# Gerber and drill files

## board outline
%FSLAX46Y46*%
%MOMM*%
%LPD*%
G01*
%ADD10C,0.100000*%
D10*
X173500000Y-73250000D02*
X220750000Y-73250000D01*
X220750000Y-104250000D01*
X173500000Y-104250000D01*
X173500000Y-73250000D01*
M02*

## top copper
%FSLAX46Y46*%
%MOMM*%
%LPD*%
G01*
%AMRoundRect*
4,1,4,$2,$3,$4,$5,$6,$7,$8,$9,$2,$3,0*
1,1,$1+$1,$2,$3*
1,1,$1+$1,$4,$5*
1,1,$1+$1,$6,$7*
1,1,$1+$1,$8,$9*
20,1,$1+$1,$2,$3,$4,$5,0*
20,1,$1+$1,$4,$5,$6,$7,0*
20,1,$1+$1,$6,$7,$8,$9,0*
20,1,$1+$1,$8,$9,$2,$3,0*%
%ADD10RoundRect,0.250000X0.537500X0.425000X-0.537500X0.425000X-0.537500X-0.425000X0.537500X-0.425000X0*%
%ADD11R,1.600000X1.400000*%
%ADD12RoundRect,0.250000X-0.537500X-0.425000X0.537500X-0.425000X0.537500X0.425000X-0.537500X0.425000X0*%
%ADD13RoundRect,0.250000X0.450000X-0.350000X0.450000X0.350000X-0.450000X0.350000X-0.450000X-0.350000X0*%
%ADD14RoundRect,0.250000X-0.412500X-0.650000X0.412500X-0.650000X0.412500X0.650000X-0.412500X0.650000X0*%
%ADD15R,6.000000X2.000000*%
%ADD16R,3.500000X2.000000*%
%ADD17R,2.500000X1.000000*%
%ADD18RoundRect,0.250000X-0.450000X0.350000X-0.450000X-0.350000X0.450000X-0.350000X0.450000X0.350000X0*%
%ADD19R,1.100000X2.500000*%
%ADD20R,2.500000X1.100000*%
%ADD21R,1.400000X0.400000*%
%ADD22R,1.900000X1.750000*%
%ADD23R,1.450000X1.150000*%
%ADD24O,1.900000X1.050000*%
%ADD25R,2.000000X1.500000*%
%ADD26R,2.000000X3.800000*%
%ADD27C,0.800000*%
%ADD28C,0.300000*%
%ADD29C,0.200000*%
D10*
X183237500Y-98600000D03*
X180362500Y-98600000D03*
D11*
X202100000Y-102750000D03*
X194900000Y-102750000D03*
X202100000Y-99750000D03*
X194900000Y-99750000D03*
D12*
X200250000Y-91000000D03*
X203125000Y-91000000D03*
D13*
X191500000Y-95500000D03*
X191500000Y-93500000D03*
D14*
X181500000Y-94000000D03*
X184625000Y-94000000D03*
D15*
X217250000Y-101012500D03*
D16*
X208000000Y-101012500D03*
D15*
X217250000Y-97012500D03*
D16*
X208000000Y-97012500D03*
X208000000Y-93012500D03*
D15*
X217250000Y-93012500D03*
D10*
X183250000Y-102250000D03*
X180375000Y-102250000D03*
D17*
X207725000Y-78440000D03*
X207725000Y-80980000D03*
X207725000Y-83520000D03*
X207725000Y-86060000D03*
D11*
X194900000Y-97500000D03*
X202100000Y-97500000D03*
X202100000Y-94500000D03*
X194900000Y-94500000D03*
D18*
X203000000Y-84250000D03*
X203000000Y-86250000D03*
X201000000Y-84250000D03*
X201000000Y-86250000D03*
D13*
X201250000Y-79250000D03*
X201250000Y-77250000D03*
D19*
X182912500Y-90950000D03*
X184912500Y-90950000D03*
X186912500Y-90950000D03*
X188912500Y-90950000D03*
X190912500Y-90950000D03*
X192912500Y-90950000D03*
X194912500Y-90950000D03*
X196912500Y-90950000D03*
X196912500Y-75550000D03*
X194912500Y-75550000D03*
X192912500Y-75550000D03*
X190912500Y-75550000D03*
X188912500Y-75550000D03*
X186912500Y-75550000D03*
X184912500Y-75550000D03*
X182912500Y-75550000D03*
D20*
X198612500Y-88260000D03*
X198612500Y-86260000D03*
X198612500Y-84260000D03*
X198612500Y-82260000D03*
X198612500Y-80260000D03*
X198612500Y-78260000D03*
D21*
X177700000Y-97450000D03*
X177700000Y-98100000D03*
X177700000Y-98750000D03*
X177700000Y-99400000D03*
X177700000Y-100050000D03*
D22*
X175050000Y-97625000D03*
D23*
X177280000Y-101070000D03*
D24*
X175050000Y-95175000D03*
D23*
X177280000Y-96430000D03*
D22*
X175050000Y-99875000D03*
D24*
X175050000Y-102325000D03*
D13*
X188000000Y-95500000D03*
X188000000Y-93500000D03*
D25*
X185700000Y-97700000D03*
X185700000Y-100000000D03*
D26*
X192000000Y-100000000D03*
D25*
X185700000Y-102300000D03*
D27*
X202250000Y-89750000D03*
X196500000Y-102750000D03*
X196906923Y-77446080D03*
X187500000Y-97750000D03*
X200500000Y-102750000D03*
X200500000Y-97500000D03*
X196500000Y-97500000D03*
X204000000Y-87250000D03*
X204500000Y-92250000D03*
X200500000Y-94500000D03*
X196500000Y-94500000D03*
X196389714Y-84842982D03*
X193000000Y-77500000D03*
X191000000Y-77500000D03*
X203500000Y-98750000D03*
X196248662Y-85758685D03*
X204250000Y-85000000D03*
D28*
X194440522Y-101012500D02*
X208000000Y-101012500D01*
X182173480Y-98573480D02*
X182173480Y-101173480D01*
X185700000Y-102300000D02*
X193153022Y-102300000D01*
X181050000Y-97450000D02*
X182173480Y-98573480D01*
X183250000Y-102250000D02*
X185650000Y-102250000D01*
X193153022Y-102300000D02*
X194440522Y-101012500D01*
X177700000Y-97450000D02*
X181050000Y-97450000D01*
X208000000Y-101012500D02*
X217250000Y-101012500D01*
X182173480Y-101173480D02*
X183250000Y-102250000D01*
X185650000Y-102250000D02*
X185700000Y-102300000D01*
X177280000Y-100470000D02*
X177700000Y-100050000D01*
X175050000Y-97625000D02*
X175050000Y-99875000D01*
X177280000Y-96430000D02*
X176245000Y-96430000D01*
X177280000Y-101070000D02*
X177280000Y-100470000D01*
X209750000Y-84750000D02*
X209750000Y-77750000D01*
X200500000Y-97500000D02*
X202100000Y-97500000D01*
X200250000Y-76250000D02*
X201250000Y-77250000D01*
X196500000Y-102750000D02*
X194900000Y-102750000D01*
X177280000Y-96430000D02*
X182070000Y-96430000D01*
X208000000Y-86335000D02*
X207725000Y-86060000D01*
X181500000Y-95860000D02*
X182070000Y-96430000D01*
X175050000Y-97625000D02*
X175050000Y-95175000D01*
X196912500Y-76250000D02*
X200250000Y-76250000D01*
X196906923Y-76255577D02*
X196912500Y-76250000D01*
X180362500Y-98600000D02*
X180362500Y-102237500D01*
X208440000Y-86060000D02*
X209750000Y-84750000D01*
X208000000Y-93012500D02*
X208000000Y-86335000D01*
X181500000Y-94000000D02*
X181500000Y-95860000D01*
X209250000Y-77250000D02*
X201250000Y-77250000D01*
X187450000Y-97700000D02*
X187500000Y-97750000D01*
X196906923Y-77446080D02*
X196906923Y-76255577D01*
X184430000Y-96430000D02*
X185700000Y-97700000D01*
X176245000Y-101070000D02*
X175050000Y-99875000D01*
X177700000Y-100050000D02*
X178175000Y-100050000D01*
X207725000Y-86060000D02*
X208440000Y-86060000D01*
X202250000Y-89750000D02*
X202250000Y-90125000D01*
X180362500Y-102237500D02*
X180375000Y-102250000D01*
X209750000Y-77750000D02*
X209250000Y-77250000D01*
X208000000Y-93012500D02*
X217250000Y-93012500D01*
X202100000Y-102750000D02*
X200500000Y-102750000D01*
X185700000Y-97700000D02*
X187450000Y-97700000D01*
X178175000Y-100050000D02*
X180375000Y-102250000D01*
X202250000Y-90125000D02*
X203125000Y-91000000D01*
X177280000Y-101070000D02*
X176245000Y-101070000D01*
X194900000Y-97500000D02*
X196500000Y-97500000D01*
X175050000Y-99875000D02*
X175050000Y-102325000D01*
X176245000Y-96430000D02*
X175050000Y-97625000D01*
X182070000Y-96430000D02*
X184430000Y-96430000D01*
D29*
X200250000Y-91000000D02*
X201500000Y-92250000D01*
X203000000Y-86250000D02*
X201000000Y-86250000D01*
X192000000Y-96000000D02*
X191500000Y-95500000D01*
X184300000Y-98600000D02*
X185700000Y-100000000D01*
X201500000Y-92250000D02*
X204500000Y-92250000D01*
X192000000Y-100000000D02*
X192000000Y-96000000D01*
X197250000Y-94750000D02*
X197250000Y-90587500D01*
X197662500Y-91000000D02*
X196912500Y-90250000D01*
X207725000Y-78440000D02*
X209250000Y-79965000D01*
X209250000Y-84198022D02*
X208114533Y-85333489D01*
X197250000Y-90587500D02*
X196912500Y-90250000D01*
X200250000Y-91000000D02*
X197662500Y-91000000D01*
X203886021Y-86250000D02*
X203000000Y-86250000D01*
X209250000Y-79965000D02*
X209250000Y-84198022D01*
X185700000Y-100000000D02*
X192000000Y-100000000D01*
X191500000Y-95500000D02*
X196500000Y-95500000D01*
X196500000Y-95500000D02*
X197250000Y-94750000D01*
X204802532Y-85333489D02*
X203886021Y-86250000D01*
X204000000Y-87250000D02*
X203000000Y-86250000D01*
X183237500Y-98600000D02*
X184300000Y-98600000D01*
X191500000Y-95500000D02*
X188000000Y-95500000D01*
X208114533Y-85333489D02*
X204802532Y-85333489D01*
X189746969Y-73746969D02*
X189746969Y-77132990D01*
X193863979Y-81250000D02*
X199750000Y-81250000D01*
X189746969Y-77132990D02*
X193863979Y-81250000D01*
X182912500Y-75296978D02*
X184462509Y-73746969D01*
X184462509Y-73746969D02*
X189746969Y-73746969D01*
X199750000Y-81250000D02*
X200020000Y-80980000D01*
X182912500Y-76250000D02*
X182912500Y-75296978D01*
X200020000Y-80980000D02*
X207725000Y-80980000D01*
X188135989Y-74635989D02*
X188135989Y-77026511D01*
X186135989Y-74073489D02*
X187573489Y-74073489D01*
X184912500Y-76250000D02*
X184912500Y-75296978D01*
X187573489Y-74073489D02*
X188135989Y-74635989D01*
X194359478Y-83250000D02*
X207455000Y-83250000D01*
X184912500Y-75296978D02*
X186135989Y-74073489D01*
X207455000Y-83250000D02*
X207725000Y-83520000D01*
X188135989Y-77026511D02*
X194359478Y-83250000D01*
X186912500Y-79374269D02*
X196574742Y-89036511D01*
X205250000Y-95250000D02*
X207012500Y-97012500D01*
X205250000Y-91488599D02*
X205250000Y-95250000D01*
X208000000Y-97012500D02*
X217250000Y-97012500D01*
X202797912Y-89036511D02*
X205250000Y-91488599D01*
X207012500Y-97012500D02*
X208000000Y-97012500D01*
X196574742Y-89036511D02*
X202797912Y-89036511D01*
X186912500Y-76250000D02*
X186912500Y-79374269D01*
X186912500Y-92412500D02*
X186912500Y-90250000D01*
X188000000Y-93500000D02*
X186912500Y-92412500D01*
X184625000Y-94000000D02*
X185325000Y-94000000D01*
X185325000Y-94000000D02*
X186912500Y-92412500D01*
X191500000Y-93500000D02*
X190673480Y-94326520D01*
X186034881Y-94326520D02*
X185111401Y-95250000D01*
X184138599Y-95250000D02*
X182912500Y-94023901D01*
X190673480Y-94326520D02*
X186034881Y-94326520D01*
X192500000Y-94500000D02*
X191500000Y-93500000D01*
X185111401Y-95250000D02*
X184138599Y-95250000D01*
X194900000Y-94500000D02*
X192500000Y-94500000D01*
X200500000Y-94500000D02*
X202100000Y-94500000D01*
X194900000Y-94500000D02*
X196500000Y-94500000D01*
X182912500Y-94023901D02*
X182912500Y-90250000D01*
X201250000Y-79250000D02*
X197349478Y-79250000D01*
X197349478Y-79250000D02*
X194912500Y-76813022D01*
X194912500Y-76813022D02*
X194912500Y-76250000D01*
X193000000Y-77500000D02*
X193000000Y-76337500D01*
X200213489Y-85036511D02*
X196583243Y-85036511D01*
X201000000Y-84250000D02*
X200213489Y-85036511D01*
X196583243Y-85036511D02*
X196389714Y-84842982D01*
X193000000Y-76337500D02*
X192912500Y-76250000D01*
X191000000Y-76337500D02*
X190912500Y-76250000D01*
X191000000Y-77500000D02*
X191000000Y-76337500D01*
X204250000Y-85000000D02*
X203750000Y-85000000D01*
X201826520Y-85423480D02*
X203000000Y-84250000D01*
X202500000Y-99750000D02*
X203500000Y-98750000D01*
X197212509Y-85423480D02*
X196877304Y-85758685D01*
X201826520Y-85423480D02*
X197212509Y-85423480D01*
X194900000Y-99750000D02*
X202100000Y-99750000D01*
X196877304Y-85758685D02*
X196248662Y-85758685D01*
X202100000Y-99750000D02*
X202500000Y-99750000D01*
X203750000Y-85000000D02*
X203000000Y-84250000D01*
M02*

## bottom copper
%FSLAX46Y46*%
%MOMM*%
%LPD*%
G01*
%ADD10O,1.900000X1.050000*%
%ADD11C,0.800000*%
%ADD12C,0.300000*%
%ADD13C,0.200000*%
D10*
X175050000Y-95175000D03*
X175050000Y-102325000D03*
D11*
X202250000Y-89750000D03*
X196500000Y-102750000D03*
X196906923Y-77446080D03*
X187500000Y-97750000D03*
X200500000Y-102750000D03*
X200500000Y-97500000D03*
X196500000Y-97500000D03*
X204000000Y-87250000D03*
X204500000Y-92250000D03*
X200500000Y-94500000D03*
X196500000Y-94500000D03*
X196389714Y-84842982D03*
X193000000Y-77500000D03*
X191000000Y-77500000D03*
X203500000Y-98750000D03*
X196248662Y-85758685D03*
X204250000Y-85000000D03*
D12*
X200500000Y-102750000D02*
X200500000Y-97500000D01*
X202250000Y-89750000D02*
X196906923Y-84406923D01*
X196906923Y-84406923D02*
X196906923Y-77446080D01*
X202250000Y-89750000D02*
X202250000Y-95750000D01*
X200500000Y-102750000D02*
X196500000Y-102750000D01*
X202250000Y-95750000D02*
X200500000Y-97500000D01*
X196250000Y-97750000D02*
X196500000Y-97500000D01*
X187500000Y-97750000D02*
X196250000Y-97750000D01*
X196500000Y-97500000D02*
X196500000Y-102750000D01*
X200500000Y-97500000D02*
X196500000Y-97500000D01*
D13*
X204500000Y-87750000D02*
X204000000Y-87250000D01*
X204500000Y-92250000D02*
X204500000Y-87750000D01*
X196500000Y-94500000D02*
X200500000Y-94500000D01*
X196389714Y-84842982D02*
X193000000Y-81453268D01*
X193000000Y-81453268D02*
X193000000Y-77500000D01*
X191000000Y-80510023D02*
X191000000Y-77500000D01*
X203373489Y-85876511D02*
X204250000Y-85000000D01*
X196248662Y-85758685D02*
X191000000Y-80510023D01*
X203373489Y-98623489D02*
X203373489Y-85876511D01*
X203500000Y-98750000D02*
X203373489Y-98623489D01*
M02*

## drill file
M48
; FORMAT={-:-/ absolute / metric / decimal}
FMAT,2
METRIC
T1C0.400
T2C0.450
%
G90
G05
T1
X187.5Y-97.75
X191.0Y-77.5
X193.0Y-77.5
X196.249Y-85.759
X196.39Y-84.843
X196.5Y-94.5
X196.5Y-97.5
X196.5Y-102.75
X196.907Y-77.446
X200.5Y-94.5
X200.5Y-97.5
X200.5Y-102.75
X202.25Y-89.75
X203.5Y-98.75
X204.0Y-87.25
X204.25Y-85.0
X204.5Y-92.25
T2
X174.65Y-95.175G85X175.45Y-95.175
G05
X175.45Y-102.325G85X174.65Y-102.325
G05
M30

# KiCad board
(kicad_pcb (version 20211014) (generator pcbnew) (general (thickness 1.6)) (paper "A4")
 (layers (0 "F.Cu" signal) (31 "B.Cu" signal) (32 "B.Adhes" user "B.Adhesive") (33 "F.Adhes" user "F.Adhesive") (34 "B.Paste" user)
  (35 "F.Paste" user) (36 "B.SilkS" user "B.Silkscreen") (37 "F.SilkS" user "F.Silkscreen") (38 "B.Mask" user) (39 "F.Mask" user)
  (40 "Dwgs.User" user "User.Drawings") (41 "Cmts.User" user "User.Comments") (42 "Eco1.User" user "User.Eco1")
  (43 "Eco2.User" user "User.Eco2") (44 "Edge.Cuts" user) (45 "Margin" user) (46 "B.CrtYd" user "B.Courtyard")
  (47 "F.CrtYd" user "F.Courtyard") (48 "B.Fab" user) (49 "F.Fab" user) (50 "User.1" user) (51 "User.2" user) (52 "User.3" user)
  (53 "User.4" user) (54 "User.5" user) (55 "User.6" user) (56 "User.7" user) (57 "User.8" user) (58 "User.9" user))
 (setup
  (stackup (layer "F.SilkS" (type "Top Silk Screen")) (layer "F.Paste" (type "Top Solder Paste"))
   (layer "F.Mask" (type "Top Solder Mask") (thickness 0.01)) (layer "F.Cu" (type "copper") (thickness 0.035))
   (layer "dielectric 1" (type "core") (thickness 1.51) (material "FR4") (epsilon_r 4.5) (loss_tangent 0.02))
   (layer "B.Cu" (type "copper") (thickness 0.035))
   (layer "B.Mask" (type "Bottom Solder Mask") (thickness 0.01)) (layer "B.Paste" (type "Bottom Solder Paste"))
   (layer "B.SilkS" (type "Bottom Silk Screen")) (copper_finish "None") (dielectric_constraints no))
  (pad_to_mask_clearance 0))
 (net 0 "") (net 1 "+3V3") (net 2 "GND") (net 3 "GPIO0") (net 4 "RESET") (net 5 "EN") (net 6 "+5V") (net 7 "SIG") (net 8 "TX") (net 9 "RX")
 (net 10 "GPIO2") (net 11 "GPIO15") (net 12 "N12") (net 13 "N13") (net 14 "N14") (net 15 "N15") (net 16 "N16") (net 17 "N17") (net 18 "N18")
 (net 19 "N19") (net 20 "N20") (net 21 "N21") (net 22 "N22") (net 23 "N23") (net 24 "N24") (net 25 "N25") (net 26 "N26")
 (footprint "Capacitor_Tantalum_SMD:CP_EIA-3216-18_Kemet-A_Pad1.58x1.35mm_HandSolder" (layer "F.Cu") (at 181.8 98.6 180)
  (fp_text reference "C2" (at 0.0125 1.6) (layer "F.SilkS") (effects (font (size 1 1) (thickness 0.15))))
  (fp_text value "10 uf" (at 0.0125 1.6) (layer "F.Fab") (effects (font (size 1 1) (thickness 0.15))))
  (pad "1" smd roundrect locked (at -1.4375 0 180) (size 1.575 1.35) (layers "F.Cu" "F.Paste" "F.Mask") (roundrect_rratio 0.1851851852)
   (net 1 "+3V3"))
  (pad "2" smd roundrect locked (at 1.4375 0 180) (size 1.575 1.35) (layers "F.Cu" "F.Paste" "F.Mask") (roundrect_rratio 0.1851851852)
   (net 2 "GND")))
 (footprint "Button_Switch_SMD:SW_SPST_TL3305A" (layer "F.Cu") (at 198.5 101.25 180)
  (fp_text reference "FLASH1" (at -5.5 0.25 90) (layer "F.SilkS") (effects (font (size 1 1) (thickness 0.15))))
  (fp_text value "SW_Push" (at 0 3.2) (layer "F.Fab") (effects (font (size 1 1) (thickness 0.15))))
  (pad "1" smd rect locked (at -3.6 -1.5 180) (size 1.6 1.4) (layers "F.Cu" "F.Paste" "F.Mask") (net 2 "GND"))
  (pad "1" smd rect locked (at 3.6 -1.5 180) (size 1.6 1.4) (layers "F.Cu" "F.Paste" "F.Mask") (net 2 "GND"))
  (pad "2" smd rect locked (at -3.6 1.5 180) (size 1.6 1.4) (layers "F.Cu" "F.Paste" "F.Mask") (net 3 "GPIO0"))
  (pad "2" smd rect locked (at 3.6 1.5 180) (size 1.6 1.4) (layers "F.Cu" "F.Paste" "F.Mask") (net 3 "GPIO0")))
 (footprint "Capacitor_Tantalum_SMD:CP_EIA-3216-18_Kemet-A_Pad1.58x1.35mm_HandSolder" (layer "F.Cu") (at 201.6875 91)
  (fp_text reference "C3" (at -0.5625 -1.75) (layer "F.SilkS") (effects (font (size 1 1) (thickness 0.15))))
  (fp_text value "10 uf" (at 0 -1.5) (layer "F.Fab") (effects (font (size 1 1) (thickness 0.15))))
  (pad "1" smd roundrect locked (at -1.4375 0) (size 1.575 1.35) (layers "F.Cu" "F.Paste" "F.Mask") (roundrect_rratio 0.1851851852)
   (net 1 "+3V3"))
  (pad "2" smd roundrect locked (at 1.4375 0) (size 1.575 1.35) (layers "F.Cu" "F.Paste" "F.Mask") (roundrect_rratio 0.1851851852)
   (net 2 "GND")))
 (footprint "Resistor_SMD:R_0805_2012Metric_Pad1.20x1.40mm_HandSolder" (layer "F.Cu") (at 191.5 94.5 90)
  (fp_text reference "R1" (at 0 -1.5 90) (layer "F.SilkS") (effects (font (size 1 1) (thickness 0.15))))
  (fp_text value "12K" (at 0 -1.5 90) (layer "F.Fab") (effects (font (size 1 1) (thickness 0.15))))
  (pad "1" smd roundrect locked (at -1 0 90) (size 1.2 1.4) (layers "F.Cu" "F.Paste" "F.Mask") (roundrect_rratio 0.2083333333)
   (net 1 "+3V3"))
  (pad "2" smd roundrect locked (at 1 0 90) (size 1.2 1.4) (layers "F.Cu" "F.Paste" "F.Mask") (roundrect_rratio 0.2083333333)
   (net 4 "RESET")))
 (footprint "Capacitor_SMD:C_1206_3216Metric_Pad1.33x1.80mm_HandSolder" (layer "F.Cu") (at 183.0625 94)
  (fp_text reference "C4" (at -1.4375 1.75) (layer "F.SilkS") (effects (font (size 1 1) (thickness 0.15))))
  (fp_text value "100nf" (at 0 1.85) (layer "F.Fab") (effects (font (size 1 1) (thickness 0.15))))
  (pad "1" smd roundrect locked (at -1.5625 0) (size 1.325 1.8) (layers "F.Cu" "F.Paste" "F.Mask") (roundrect_rratio 0.1886792453)
   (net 2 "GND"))
  (pad "2" smd roundrect locked (at 1.5625 0) (size 1.325 1.8) (layers "F.Cu" "F.Paste" "F.Mask") (roundrect_rratio 0.1886792453)
   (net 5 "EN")))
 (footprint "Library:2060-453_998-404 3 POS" (layer "F.Cu") (at 212.25 105.0125 180)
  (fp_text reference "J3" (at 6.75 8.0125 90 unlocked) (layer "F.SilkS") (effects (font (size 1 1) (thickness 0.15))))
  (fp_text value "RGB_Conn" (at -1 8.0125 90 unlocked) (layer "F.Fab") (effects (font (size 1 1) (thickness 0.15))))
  (pad "1" smd rect (at -5 4 180) (size 6 2) (layers "F.Cu" "F.Paste" "F.Mask") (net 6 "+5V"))
  (pad "1" smd rect (at 4.25 4 180) (size 3.5 2) (layers "F.Cu" "F.Paste" "F.Mask") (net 6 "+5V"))
  (pad "2" smd rect (at -5 8 180) (size 6 2) (layers "F.Cu" "F.Paste" "F.Mask") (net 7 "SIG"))
  (pad "2" smd rect (at 4.25 8 180) (size 3.5 2) (layers "F.Cu" "F.Paste" "F.Mask") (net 7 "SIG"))
  (pad "3" smd rect (at 4.25 12 180) (size 3.5 2) (layers "F.Cu" "F.Paste" "F.Mask") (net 2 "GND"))
  (pad "3" smd rect (at -5 12 180) (size 6 2) (layers "F.Cu" "F.Paste" "F.Mask") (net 2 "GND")))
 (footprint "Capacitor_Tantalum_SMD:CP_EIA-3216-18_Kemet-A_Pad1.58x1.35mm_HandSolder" (layer "F.Cu") (at 181.8125 102.25 180)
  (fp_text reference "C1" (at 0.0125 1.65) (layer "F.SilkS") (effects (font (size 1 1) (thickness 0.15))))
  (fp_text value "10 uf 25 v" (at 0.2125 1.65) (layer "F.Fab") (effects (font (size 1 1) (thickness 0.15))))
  (pad "1" smd roundrect locked (at -1.4375 0 180) (size 1.575 1.35) (layers "F.Cu" "F.Paste" "F.Mask") (roundrect_rratio 0.1851851852)
   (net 6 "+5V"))
  (pad "2" smd roundrect locked (at 1.4375 0 180) (size 1.575 1.35) (layers "F.Cu" "F.Paste" "F.Mask") (roundrect_rratio 0.1851851852)
   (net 2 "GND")))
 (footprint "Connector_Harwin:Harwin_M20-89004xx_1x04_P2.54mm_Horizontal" (layer "F.Cu") (at 213.25 82.25)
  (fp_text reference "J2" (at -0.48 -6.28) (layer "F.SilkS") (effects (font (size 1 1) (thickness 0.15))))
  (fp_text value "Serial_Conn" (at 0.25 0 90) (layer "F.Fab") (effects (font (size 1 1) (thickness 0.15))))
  (pad "" smd rect (at 3.895 -3.81) (size 5.7 0.6) (layers "F.SilkS"))
  (pad "1" smd rect (at -5.525 -3.81) (size 2.5 1) (layers "F.Cu" "F.Paste" "F.Mask") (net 1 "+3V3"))
  (pad "2" smd rect (at -5.525 -1.27) (size 2.5 1) (layers "F.Cu" "F.Paste" "F.Mask") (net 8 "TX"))
  (pad "3" smd rect (at -5.525 1.27) (size 2.5 1) (layers "F.Cu" "F.Paste" "F.Mask") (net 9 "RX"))
  (pad "4" smd rect (at -5.525 3.81) (size 2.5 1) (layers "F.Cu" "F.Paste" "F.Mask") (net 2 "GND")))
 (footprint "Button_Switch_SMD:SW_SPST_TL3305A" (layer "F.Cu") (at 198.5 96 180)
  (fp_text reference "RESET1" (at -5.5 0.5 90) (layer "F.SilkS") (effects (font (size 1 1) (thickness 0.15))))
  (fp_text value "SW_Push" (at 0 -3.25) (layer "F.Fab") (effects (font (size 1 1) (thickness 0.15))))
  (pad "1" smd rect locked (at 3.6 -1.5 180) (size 1.6 1.4) (layers "F.Cu" "F.Paste" "F.Mask") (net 2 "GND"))
  (pad "1" smd rect locked (at -3.6 -1.5 180) (size 1.6 1.4) (layers "F.Cu" "F.Paste" "F.Mask") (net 2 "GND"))
  (pad "2" smd rect locked (at -3.6 1.5 180) (size 1.6 1.4) (layers "F.Cu" "F.Paste" "F.Mask") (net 4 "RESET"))
  (pad "2" smd rect locked (at 3.6 1.5 180) (size 1.6 1.4) (layers "F.Cu" "F.Paste" "F.Mask") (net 4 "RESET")))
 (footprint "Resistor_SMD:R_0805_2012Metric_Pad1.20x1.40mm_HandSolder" (layer "F.Cu") (at 203 85.25 -90)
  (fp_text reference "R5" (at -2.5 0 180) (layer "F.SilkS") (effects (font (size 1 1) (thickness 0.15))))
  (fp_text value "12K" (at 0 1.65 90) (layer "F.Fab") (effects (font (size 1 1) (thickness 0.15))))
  (pad "1" smd roundrect locked (at -1 0 270) (size 1.2 1.4) (layers "F.Cu" "F.Paste" "F.Mask") (roundrect_rratio 0.2083333333)
   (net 3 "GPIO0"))
  (pad "2" smd roundrect locked (at 1 0 270) (size 1.2 1.4) (layers "F.Cu" "F.Paste" "F.Mask") (roundrect_rratio 0.2083333333)
   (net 1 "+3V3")))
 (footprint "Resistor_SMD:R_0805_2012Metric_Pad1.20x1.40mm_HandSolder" (layer "F.Cu") (at 201 85.25 -90)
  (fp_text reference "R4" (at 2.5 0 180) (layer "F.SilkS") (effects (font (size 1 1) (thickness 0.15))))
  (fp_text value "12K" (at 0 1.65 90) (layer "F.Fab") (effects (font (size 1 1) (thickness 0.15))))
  (pad "1" smd roundrect locked (at -1 0 270) (size 1.2 1.4) (layers "F.Cu" "F.Paste" "F.Mask") (roundrect_rratio 0.2083333333)
   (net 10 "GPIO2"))
  (pad "2" smd roundrect locked (at 1 0 270) (size 1.2 1.4) (layers "F.Cu" "F.Paste" "F.Mask") (roundrect_rratio 0.2083333333)
   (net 1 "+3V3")))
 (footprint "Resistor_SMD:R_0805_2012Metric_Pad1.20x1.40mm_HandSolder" (layer "F.Cu") (at 201.25 78.25 90)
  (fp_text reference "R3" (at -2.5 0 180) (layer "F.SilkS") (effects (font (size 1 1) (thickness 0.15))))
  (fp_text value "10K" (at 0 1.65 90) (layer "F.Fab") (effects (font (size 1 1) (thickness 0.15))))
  (pad "1" smd roundrect locked (at -1 0 90) (size 1.2 1.4) (layers "F.Cu" "F.Paste" "F.Mask") (roundrect_rratio 0.2083333333)
   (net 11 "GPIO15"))
  (pad "2" smd roundrect locked (at 1 0 90) (size 1.2 1.4) (layers "F.Cu" "F.Paste" "F.Mask") (roundrect_rratio 0.2083333333) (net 2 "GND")))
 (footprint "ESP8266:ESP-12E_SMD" (layer "F.Cu") (at 182.9125 90.25 90)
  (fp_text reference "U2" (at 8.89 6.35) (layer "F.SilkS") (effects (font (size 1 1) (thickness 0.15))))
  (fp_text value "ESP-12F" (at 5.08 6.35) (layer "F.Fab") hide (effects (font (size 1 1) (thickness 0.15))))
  (pad "1" smd rect (at 0 0 90) (size 2.5 1.1) (drill (offset -0.7 0)) (layers "F.Cu" "F.Paste" "F.Mask") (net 4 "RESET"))
  (pad "2" smd rect (at 0 2 90) (size 2.5 1.1) (drill (offset -0.7 0)) (layers "F.Cu" "F.Paste" "F.Mask") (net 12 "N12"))
  (pad "3" smd rect (at 0 4 90) (size 2.5 1.1) (drill (offset -0.7 0)) (layers "F.Cu" "F.Paste" "F.Mask") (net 5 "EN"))
  (pad "4" smd rect (at 0 6 90) (size 2.5 1.1) (drill (offset -0.7 0)) (layers "F.Cu" "F.Paste" "F.Mask") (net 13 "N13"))
  (pad "5" smd rect (at 0 8 90) (size 2.5 1.1) (drill (offset -0.7 0)) (layers "F.Cu" "F.Paste" "F.Mask") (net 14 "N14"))
  (pad "6" smd rect (at 0 10 90) (size 2.5 1.1) (drill (offset -0.7 0)) (layers "F.Cu" "F.Paste" "F.Mask") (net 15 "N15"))
  (pad "7" smd rect (at 0 12 90) (size 2.5 1.1) (drill (offset -0.7 0)) (layers "F.Cu" "F.Paste" "F.Mask") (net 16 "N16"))
  (pad "8" smd rect (at 0 14 90) (size 2.5 1.1) (drill (offset -0.7 0)) (layers "F.Cu" "F.Paste" "F.Mask") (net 1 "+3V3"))
  (pad "9" smd rect (at 14 14 90) (size 2.5 1.1) (drill (offset 0.7 0)) (layers "F.Cu" "F.Paste" "F.Mask") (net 2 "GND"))
  (pad "10" smd rect (at 14 12 90) (size 2.5 1.1) (drill (offset 0.7 0)) (layers "F.Cu" "F.Paste" "F.Mask") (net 11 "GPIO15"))
  (pad "11" smd rect (at 14 10 90) (size 2.5 1.1) (drill (offset 0.7 0)) (layers "F.Cu" "F.Paste" "F.Mask") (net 10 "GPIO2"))
  (pad "12" smd rect (at 14 8 90) (size 2.5 1.1) (drill (offset 0.7 0)) (layers "F.Cu" "F.Paste" "F.Mask") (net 3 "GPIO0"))
  (pad "13" smd rect (at 14 6 90) (size 2.5 1.1) (drill (offset 0.7 0)) (layers "F.Cu" "F.Paste" "F.Mask") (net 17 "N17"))
  (pad "14" smd rect (at 14 4 90) (size 2.5 1.1) (drill (offset 0.7 0)) (layers "F.Cu" "F.Paste" "F.Mask") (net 7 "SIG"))
  (pad "15" smd rect (at 14 2 90) (size 2.5 1.1) (drill (offset 0.7 0)) (layers "F.Cu" "F.Paste" "F.Mask") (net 9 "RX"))
  (pad "16" smd rect (at 14 0 90) (size 2.5 1.1) (drill (offset 0.7 0)) (layers "F.Cu" "F.Paste" "F.Mask") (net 8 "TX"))
  (pad "17" smd rect (at 1.99 15 180) (size 2.5 1.1) (drill (offset -0.7 0)) (layers "F.Cu" "F.Paste" "F.Mask") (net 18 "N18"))
  (pad "18" smd rect (at 3.99 15 180) (size 2.5 1.1) (drill (offset -0.7 0)) (layers "F.Cu" "F.Paste" "F.Mask") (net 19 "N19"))
  (pad "19" smd rect (at 5.99 15 180) (size 2.5 1.1) (drill (offset -0.7 0)) (layers "F.Cu" "F.Paste" "F.Mask") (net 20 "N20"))
  (pad "20" smd rect (at 7.99 15 180) (size 2.5 1.1) (drill (offset -0.7 0)) (layers "F.Cu" "F.Paste" "F.Mask") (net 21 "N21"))
  (pad "21" smd rect (at 9.99 15 180) (size 2.5 1.1) (drill (offset -0.7 0)) (layers "F.Cu" "F.Paste" "F.Mask") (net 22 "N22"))
  (pad "22" smd rect (at 11.99 15 180) (size 2.5 1.1) (drill (offset -0.7 0)) (layers "F.Cu" "F.Paste" "F.Mask") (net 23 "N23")))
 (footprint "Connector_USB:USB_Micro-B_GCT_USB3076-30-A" (layer "F.Cu") (at 176.25 98.75 -90)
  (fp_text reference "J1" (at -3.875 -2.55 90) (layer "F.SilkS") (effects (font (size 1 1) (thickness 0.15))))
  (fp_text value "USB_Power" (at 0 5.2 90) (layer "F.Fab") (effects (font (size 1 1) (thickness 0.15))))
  (pad "1" smd rect locked (at -1.3 -1.45 270) (size 0.4 1.4) (layers "F.Cu" "F.Paste" "F.Mask") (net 6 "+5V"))
  (pad "2" smd rect locked (at -0.65 -1.45 270) (size 0.4 1.4) (layers "F.Cu" "F.Paste" "F.Mask") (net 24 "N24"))
  (pad "3" smd rect locked (at 0 -1.45 270) (size 0.4 1.4) (layers "F.Cu" "F.Paste" "F.Mask") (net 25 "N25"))
  (pad "4" smd rect locked (at 0.65 -1.45 270) (size 0.4 1.4) (layers "F.Cu" "F.Paste" "F.Mask") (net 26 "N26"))
  (pad "5" smd rect locked (at 1.3 -1.45 270) (size 0.4 1.4) (layers "F.Cu" "F.Paste" "F.Mask") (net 2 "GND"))
  (pad "6" smd rect locked (at -1.125 1.2 270) (size 1.75 1.9) (layers "F.Cu" "F.Paste" "F.Mask") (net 2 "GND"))
  (pad "6" smd rect locked (at 2.32 -1.03 270) (size 1.15 1.45) (layers "F.Cu" "F.Paste" "F.Mask") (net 2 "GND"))
  (pad "6" thru_hole oval locked (at -3.575 1.2 90) (size 1.05 1.9) (drill oval 0.45 1.25) (layers *.Cu *.Mask) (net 2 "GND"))
  (pad "6" smd rect locked (at -2.32 -1.03 270) (size 1.15 1.45) (layers "F.Cu" "F.Paste" "F.Mask") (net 2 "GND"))
  (pad "6" smd rect locked (at 1.125 1.2 270) (size 1.75 1.9) (layers "F.Cu" "F.Paste" "F.Mask") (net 2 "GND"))
  (pad "6" thru_hole oval locked (at 3.575 1.2 270) (size 1.05 1.9) (drill oval 0.45 1.25) (layers *.Cu *.Mask) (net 2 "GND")))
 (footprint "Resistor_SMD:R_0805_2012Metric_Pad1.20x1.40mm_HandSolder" (layer "F.Cu") (at 188 94.5 90)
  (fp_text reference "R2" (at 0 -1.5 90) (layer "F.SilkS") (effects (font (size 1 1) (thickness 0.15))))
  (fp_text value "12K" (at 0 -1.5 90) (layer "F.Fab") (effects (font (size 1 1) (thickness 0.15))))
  (pad "1" smd roundrect locked (at -1 0 90) (size 1.2 1.4) (layers "F.Cu" "F.Paste" "F.Mask") (roundrect_rratio 0.2083333333)
   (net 1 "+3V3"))
  (pad "2" smd roundrect locked (at 1 0 90) (size 1.2 1.4) (layers "F.Cu" "F.Paste" "F.Mask") (roundrect_rratio 0.2083333333) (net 5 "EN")))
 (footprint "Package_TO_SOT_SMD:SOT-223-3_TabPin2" (layer "F.Cu") (at 188.85 100)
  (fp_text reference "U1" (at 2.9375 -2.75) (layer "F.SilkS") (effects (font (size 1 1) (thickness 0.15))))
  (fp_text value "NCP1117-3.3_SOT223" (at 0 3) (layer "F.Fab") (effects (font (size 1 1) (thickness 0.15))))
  (pad "1" smd rect locked (at -3.15 -2.3) (size 2 1.5) (layers "F.Cu" "F.Paste" "F.Mask") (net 2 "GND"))
  (pad "2" smd rect locked (at -3.15 0) (size 2 1.5) (layers "F.Cu" "F.Paste" "F.Mask") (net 1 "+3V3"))
  (pad "2" smd rect locked (at 3.15 0) (size 2 3.8) (layers "F.Cu" "F.Paste" "F.Mask") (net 1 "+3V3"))
  (pad "3" smd rect locked (at -3.15 2.3) (size 2 1.5) (layers "F.Cu" "F.Paste" "F.Mask") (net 6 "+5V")))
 (gr_rect (start 220.75 104.25) (end 173.5 73.25) (layer "Edge.Cuts") (width 0.1) (fill none))
 (segment (start 194.440522 101.0125) (end 208 101.0125) (width 0.3) (layer "F.Cu") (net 6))
 (segment (start 182.17348 98.57348) (end 182.17348 101.17348) (width 0.3) (layer "F.Cu") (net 6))
 (segment (start 185.7 102.3) (end 193.153022 102.3) (width 0.3) (layer "F.Cu") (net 6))
 (segment (start 181.05 97.45) (end 182.17348 98.57348) (width 0.3) (layer "F.Cu") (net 6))
 (segment (start 183.25 102.25) (end 185.65 102.25) (width 0.3) (layer "F.Cu") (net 6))
 (segment (start 193.153022 102.3) (end 194.440522 101.0125) (width 0.3) (layer "F.Cu") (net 6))
 (segment (start 177.7 97.45) (end 181.05 97.45) (width 0.3) (layer "F.Cu") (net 6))
 (segment (start 208 101.0125) (end 217.25 101.0125) (width 0.3) (layer "F.Cu") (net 6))
 (segment (start 182.17348 101.17348) (end 183.25 102.25) (width 0.3) (layer "F.Cu") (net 6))
 (segment (start 185.65 102.25) (end 185.7 102.3) (width 0.3) (layer "F.Cu") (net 6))
 (segment (start 177.28 100.47) (end 177.7 100.05) (width 0.3) (layer "F.Cu") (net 2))
 (segment (start 175.05 97.625) (end 175.05 99.875) (width 0.3) (layer "F.Cu") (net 2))
 (segment (start 177.28 96.43) (end 176.245 96.43) (width 0.3) (layer "F.Cu") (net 2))
 (segment (start 177.28 101.07) (end 177.28 100.47) (width 0.3) (layer "F.Cu") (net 2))
 (segment (start 209.75 84.75) (end 209.75 77.75) (width 0.3) (layer "F.Cu") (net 2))
 (segment (start 200.5 97.5) (end 202.1 97.5) (width 0.3) (layer "F.Cu") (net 2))
 (segment (start 200.25 76.25) (end 201.25 77.25) (width 0.3) (layer "F.Cu") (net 2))
 (segment (start 196.5 102.75) (end 194.9 102.75) (width 0.3) (layer "F.Cu") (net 2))
 (segment (start 177.28 96.43) (end 182.07 96.43) (width 0.3) (layer "F.Cu") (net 2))
 (segment (start 208 86.335) (end 207.725 86.06) (width 0.3) (layer "F.Cu") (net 2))
 (segment (start 181.5 95.86) (end 182.07 96.43) (width 0.3) (layer "F.Cu") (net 2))
 (segment (start 175.05 97.625) (end 175.05 95.175) (width 0.3) (layer "F.Cu") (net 2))
 (segment (start 196.9125 76.25) (end 200.25 76.25) (width 0.3) (layer "F.Cu") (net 2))
 (segment (start 196.906923 76.255577) (end 196.9125 76.25) (width 0.3) (layer "F.Cu") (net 2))
 (segment (start 180.3625 98.6) (end 180.3625 102.2375) (width 0.3) (layer "F.Cu") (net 2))
 (segment (start 208.44 86.06) (end 209.75 84.75) (width 0.3) (layer "F.Cu") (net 2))
 (segment (start 208 93.0125) (end 208 86.335) (width 0.3) (layer "F.Cu") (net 2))
 (segment (start 181.5 94) (end 181.5 95.86) (width 0.3) (layer "F.Cu") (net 2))
 (segment (start 209.25 77.25) (end 201.25 77.25) (width 0.3) (layer "F.Cu") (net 2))
 (segment (start 187.45 97.7) (end 187.5 97.75) (width 0.3) (layer "F.Cu") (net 2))
 (segment (start 196.906923 77.44608) (end 196.906923 76.255577) (width 0.3) (layer "F.Cu") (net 2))
 (segment (start 184.43 96.43) (end 185.7 97.7) (width 0.3) (layer "F.Cu") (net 2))
 (segment (start 176.245 101.07) (end 175.05 99.875) (width 0.3) (layer "F.Cu") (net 2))
 (segment (start 177.7 100.05) (end 178.175 100.05) (width 0.3) (layer "F.Cu") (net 2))
 (segment (start 207.725 86.06) (end 208.44 86.06) (width 0.3) (layer "F.Cu") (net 2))
 (segment (start 202.25 89.75) (end 202.25 90.125) (width 0.3) (layer "F.Cu") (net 2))
 (segment (start 180.3625 102.2375) (end 180.375 102.25) (width 0.3) (layer "F.Cu") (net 2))
 (segment (start 209.75 77.75) (end 209.25 77.25) (width 0.3) (layer "F.Cu") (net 2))
 (segment (start 208 93.0125) (end 217.25 93.0125) (width 0.3) (layer "F.Cu") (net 2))
 (segment (start 202.1 102.75) (end 200.5 102.75) (width 0.3) (layer "F.Cu") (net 2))
 (segment (start 185.7 97.7) (end 187.45 97.7) (width 0.3) (layer "F.Cu") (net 2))
 (segment (start 178.175 100.05) (end 180.375 102.25) (width 0.3) (layer "F.Cu") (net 2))
 (segment (start 202.25 90.125) (end 203.125 91) (width 0.3) (layer "F.Cu") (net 2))
 (segment (start 177.28 101.07) (end 176.245 101.07) (width 0.3) (layer "F.Cu") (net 2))
 (segment (start 194.9 97.5) (end 196.5 97.5) (width 0.3) (layer "F.Cu") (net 2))
 (segment (start 175.05 99.875) (end 175.05 102.325) (width 0.3) (layer "F.Cu") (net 2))
 (segment (start 176.245 96.43) (end 175.05 97.625) (width 0.3) (layer "F.Cu") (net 2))
 (segment (start 182.07 96.43) (end 184.43 96.43) (width 0.3) (layer "F.Cu") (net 2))
 (via (at 202.25 89.75) (size 0.8) (drill 0.4) (layers "F.Cu" "B.Cu") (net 2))
 (via (at 196.5 102.75) (size 0.8) (drill 0.4) (layers "F.Cu" "B.Cu") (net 2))
 (via (at 196.906923 77.44608) (size 0.8) (drill 0.4) (layers "F.Cu" "B.Cu") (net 2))
 (via (at 187.5 97.75) (size 0.8) (drill 0.4) (layers "F.Cu" "B.Cu") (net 2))
 (via (at 200.5 102.75) (size 0.8) (drill 0.4) (layers "F.Cu" "B.Cu") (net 2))
 (via (at 200.5 97.5) (size 0.8) (drill 0.4) (layers "F.Cu" "B.Cu") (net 2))
 (via (at 196.5 97.5) (size 0.8) (drill 0.4) (layers "F.Cu" "B.Cu") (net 2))
 (segment (start 200.5 102.75) (end 200.5 97.5) (width 0.3) (layer "B.Cu") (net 2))
 (segment (start 202.25 89.75) (end 196.906923 84.406923) (width 0.3) (layer "B.Cu") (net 2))
 (segment (start 196.906923 84.406923) (end 196.906923 77.44608) (width 0.3) (layer "B.Cu") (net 2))
 (segment (start 202.25 89.75) (end 202.25 95.75) (width 0.3) (layer "B.Cu") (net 2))
 (segment (start 200.5 102.75) (end 196.5 102.75) (width 0.3) (layer "B.Cu") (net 2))
 (segment (start 202.25 95.75) (end 200.5 97.5) (width 0.3) (layer "B.Cu") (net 2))
 (segment (start 196.25 97.75) (end 196.5 97.5) (width 0.3) (layer "B.Cu") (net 2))
 (segment (start 187.5 97.75) (end 196.25 97.75) (width 0.3) (layer "B.Cu") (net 2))
 (segment (start 196.5 97.5) (end 196.5 102.75) (width 0.3) (layer "B.Cu") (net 2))
 (segment (start 200.5 97.5) (end 196.5 97.5) (width 0.3) (layer "B.Cu") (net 2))
 (segment (start 200.25 91) (end 201.5 92.25) (width 0.2) (layer "F.Cu") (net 1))
 (segment (start 203 86.25) (end 201 86.25) (width 0.2) (layer "F.Cu") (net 1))
 (segment (start 192 96) (end 191.5 95.5) (width 0.2) (layer "F.Cu") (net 1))
 (segment (start 184.3 98.6) (end 185.7 100) (width 0.2) (layer "F.Cu") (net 1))
 (segment (start 201.5 92.25) (end 204.5 92.25) (width 0.2) (layer "F.Cu") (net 1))
 (segment (start 192 100) (end 192 96) (width 0.2) (layer "F.Cu") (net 1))
 (segment (start 197.25 94.75) (end 197.25 90.5875) (width 0.2) (layer "F.Cu") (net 1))
 (segment (start 197.6625 91) (end 196.9125 90.25) (width 0.2) (layer "F.Cu") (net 1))
 (segment (start 207.725 78.44) (end 209.25 79.965) (width 0.2) (layer "F.Cu") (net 1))
 (segment (start 209.25 84.198022) (end 208.114533 85.333489) (width 0.2) (layer "F.Cu") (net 1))
 (segment (start 197.25 90.5875) (end 196.9125 90.25) (width 0.2) (layer "F.Cu") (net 1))
 (segment (start 200.25 91) (end 197.6625 91) (width 0.2) (layer "F.Cu") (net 1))
 (segment (start 203.886021 86.25) (end 203 86.25) (width 0.2) (layer "F.Cu") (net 1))
 (segment (start 209.25 79.965) (end 209.25 84.198022) (width 0.2) (layer "F.Cu") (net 1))
 (segment (start 185.7 100) (end 192 100) (width 0.2) (layer "F.Cu") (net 1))
 (segment (start 191.5 95.5) (end 196.5 95.5) (width 0.2) (layer "F.Cu") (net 1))
 (segment (start 196.5 95.5) (end 197.25 94.75) (width 0.2) (layer "F.Cu") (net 1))
 (segment (start 204.802532 85.333489) (end 203.886021 86.25) (width 0.2) (layer "F.Cu") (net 1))
 (segment (start 204 87.25) (end 203 86.25) (width 0.2) (layer "F.Cu") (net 1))
 (segment (start 183.2375 98.6) (end 184.3 98.6) (width 0.2) (layer "F.Cu") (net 1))
 (segment (start 191.5 95.5) (end 188 95.5) (width 0.2) (layer "F.Cu") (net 1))
 (segment (start 208.114533 85.333489) (end 204.802532 85.333489) (width 0.2) (layer "F.Cu") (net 1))
 (via (at 204 87.25) (size 0.8) (drill 0.4) (layers "F.Cu" "B.Cu") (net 1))
 (via (at 204.5 92.25) (size 0.8) (drill 0.4) (layers "F.Cu" "B.Cu") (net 1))
 (segment (start 204.5 87.75) (end 204 87.25) (width 0.2) (layer "B.Cu") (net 1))
 (segment (start 204.5 92.25) (end 204.5 87.75) (width 0.2) (layer "B.Cu") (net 1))
 (segment (start 189.746969 73.746969) (end 189.746969 77.13299) (width 0.2) (layer "F.Cu") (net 8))
 (segment (start 193.863979 81.25) (end 199.75 81.25) (width 0.2) (layer "F.Cu") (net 8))
 (segment (start 189.746969 77.13299) (end 193.863979 81.25) (width 0.2) (layer "F.Cu") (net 8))
 (segment (start 182.9125 75.296978) (end 184.462509 73.746969) (width 0.2) (layer "F.Cu") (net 8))
 (segment (start 184.462509 73.746969) (end 189.746969 73.746969) (width 0.2) (layer "F.Cu") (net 8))
 (segment (start 199.75 81.25) (end 200.02 80.98) (width 0.2) (layer "F.Cu") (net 8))
 (segment (start 182.9125 76.25) (end 182.9125 75.296978) (width 0.2) (layer "F.Cu") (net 8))
 (segment (start 200.02 80.98) (end 207.725 80.98) (width 0.2) (layer "F.Cu") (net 8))
 (segment (start 188.135989 74.635989) (end 188.135989 77.026511) (width 0.2) (layer "F.Cu") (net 9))
 (segment (start 186.135989 74.073489) (end 187.573489 74.073489) (width 0.2) (layer "F.Cu") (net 9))
 (segment (start 184.9125 76.25) (end 184.9125 75.296978) (width 0.2) (layer "F.Cu") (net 9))
 (segment (start 187.573489 74.073489) (end 188.135989 74.635989) (width 0.2) (layer "F.Cu") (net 9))
 (segment (start 194.359478 83.25) (end 207.455 83.25) (width 0.2) (layer "F.Cu") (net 9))
 (segment (start 184.9125 75.296978) (end 186.135989 74.073489) (width 0.2) (layer "F.Cu") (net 9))
 (segment (start 207.455 83.25) (end 207.725 83.52) (width 0.2) (layer "F.Cu") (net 9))
 (segment (start 188.135989 77.026511) (end 194.359478 83.25) (width 0.2) (layer "F.Cu") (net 9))
 (segment (start 186.9125 79.374269) (end 196.574742 89.036511) (width 0.2) (layer "F.Cu") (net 7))
 (segment (start 205.25 95.25) (end 207.0125 97.0125) (width 0.2) (layer "F.Cu") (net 7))
 (segment (start 205.25 91.488599) (end 205.25 95.25) (width 0.2) (layer "F.Cu") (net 7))
 (segment (start 208 97.0125) (end 217.25 97.0125) (width 0.2) (layer "F.Cu") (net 7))
 (segment (start 202.797912 89.036511) (end 205.25 91.488599) (width 0.2) (layer "F.Cu") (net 7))
 (segment (start 207.0125 97.0125) (end 208 97.0125) (width 0.2) (layer "F.Cu") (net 7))
 (segment (start 196.574742 89.036511) (end 202.797912 89.036511) (width 0.2) (layer "F.Cu") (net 7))
 (segment (start 186.9125 76.25) (end 186.9125 79.374269) (width 0.2) (layer "F.Cu") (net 7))
 (segment (start 186.9125 92.4125) (end 186.9125 90.25) (width 0.2) (layer "F.Cu") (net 5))
 (segment (start 188 93.5) (end 186.9125 92.4125) (width 0.2) (layer "F.Cu") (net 5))
 (segment (start 184.625 94) (end 185.325 94) (width 0.2) (layer "F.Cu") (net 5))
 (segment (start 185.325 94) (end 186.9125 92.4125) (width 0.2) (layer "F.Cu") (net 5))
 (segment (start 191.5 93.5) (end 190.67348 94.32652) (width 0.2) (layer "F.Cu") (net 4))
 (segment (start 186.034881 94.32652) (end 185.111401 95.25) (width 0.2) (layer "F.Cu") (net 4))
 (segment (start 184.138599 95.25) (end 182.9125 94.023901) (width 0.2) (layer "F.Cu") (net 4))
 (segment (start 190.67348 94.32652) (end 186.034881 94.32652) (width 0.2) (layer "F.Cu") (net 4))
 (segment (start 192.5 94.5) (end 191.5 93.5) (width 0.2) (layer "F.Cu") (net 4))
 (segment (start 185.111401 95.25) (end 184.138599 95.25) (width 0.2) (layer "F.Cu") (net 4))
 (segment (start 194.9 94.5) (end 192.5 94.5) (width 0.2) (layer "F.Cu") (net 4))
 (segment (start 200.5 94.5) (end 202.1 94.5) (width 0.2) (layer "F.Cu") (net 4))
 (segment (start 194.9 94.5) (end 196.5 94.5) (width 0.2) (layer "F.Cu") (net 4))
 (segment (start 182.9125 94.023901) (end 182.9125 90.25) (width 0.2) (layer "F.Cu") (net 4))
 (via (at 200.5 94.5) (size 0.8) (drill 0.4) (layers "F.Cu" "B.Cu") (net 4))
 (via (at 196.5 94.5) (size 0.8) (drill 0.4) (layers "F.Cu" "B.Cu") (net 4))
 (segment (start 196.5 94.5) (end 200.5 94.5) (width 0.2) (layer "B.Cu") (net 4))
 (segment (start 201.25 79.25) (end 197.349478 79.25) (width 0.2) (layer "F.Cu") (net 11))
 (segment (start 197.349478 79.25) (end 194.9125 76.813022) (width 0.2) (layer "F.Cu") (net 11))
 (segment (start 194.9125 76.813022) (end 194.9125 76.25) (width 0.2) (layer "F.Cu") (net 11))
 (segment (start 193 77.5) (end 193 76.3375) (width 0.2) (layer "F.Cu") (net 10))
 (segment (start 200.213489 85.036511) (end 196.583243 85.036511) (width 0.2) (layer "F.Cu") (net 10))
 (segment (start 201 84.25) (end 200.213489 85.036511) (width 0.2) (layer "F.Cu") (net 10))
 (segment (start 196.583243 85.036511) (end 196.389714 84.842982) (width 0.2) (layer "F.Cu") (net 10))
 (segment (start 193 76.3375) (end 192.9125 76.25) (width 0.2) (layer "F.Cu") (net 10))
 (via (at 196.389714 84.842982) (size 0.8) (drill 0.4) (layers "F.Cu" "B.Cu") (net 10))
 (via (at 193 77.5) (size 0.8) (drill 0.4) (layers "F.Cu" "B.Cu") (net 10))
 (segment (start 196.389714 84.842982) (end 193 81.453268) (width 0.2) (layer "B.Cu") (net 10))
 (segment (start 193 81.453268) (end 193 77.5) (width 0.2) (layer "B.Cu") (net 10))
 (segment (start 191 76.3375) (end 190.9125 76.25) (width 0.2) (layer "F.Cu") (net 3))
 (segment (start 191 77.5) (end 191 76.3375) (width 0.2) (layer "F.Cu") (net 3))
 (segment (start 204.25 85) (end 203.75 85) (width 0.2) (layer "F.Cu") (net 3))
 (segment (start 201.82652 85.42348) (end 203 84.25) (width 0.2) (layer "F.Cu") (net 3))
 (segment (start 202.5 99.75) (end 203.5 98.75) (width 0.2) (layer "F.Cu") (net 3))
 (segment (start 197.212509 85.42348) (end 196.877304 85.758685) (width 0.2) (layer "F.Cu") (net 3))
 (segment (start 201.82652 85.42348) (end 197.212509 85.42348) (width 0.2) (layer "F.Cu") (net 3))
 (segment (start 194.9 99.75) (end 202.1 99.75) (width 0.2) (layer "F.Cu") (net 3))
 (segment (start 196.877304 85.758685) (end 196.248662 85.758685) (width 0.2) (layer "F.Cu") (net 3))
 (segment (start 202.1 99.75) (end 202.5 99.75) (width 0.2) (layer "F.Cu") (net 3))
 (segment (start 203.75 85) (end 203 84.25) (width 0.2) (layer "F.Cu") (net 3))
 (via (at 191 77.5) (size 0.8) (drill 0.4) (layers "F.Cu" "B.Cu") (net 3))
 (via (at 203.5 98.75) (size 0.8) (drill 0.4) (layers "F.Cu" "B.Cu") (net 3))
 (via (at 196.248662 85.758685) (size 0.8) (drill 0.4) (layers "F.Cu" "B.Cu") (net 3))
 (via (at 204.25 85) (size 0.8) (drill 0.4) (layers "F.Cu" "B.Cu") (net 3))
 (segment (start 191 80.510023) (end 191 77.5) (width 0.2) (layer "B.Cu") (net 3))
 (segment (start 203.373489 85.876511) (end 204.25 85) (width 0.2) (layer "B.Cu") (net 3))
 (segment (start 196.248662 85.758685) (end 191 80.510023) (width 0.2) (layer "B.Cu") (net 3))
 (segment (start 203.373489 98.623489) (end 203.373489 85.876511) (width 0.2) (layer "B.Cu") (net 3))
 (segment (start 203.5 98.75) (end 203.373489 98.623489) (width 0.2) (layer "B.Cu") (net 3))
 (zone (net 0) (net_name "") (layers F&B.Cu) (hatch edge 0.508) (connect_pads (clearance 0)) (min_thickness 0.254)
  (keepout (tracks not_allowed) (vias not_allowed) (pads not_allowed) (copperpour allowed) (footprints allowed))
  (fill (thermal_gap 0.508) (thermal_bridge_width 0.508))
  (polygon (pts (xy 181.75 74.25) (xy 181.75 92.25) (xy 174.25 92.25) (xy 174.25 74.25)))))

